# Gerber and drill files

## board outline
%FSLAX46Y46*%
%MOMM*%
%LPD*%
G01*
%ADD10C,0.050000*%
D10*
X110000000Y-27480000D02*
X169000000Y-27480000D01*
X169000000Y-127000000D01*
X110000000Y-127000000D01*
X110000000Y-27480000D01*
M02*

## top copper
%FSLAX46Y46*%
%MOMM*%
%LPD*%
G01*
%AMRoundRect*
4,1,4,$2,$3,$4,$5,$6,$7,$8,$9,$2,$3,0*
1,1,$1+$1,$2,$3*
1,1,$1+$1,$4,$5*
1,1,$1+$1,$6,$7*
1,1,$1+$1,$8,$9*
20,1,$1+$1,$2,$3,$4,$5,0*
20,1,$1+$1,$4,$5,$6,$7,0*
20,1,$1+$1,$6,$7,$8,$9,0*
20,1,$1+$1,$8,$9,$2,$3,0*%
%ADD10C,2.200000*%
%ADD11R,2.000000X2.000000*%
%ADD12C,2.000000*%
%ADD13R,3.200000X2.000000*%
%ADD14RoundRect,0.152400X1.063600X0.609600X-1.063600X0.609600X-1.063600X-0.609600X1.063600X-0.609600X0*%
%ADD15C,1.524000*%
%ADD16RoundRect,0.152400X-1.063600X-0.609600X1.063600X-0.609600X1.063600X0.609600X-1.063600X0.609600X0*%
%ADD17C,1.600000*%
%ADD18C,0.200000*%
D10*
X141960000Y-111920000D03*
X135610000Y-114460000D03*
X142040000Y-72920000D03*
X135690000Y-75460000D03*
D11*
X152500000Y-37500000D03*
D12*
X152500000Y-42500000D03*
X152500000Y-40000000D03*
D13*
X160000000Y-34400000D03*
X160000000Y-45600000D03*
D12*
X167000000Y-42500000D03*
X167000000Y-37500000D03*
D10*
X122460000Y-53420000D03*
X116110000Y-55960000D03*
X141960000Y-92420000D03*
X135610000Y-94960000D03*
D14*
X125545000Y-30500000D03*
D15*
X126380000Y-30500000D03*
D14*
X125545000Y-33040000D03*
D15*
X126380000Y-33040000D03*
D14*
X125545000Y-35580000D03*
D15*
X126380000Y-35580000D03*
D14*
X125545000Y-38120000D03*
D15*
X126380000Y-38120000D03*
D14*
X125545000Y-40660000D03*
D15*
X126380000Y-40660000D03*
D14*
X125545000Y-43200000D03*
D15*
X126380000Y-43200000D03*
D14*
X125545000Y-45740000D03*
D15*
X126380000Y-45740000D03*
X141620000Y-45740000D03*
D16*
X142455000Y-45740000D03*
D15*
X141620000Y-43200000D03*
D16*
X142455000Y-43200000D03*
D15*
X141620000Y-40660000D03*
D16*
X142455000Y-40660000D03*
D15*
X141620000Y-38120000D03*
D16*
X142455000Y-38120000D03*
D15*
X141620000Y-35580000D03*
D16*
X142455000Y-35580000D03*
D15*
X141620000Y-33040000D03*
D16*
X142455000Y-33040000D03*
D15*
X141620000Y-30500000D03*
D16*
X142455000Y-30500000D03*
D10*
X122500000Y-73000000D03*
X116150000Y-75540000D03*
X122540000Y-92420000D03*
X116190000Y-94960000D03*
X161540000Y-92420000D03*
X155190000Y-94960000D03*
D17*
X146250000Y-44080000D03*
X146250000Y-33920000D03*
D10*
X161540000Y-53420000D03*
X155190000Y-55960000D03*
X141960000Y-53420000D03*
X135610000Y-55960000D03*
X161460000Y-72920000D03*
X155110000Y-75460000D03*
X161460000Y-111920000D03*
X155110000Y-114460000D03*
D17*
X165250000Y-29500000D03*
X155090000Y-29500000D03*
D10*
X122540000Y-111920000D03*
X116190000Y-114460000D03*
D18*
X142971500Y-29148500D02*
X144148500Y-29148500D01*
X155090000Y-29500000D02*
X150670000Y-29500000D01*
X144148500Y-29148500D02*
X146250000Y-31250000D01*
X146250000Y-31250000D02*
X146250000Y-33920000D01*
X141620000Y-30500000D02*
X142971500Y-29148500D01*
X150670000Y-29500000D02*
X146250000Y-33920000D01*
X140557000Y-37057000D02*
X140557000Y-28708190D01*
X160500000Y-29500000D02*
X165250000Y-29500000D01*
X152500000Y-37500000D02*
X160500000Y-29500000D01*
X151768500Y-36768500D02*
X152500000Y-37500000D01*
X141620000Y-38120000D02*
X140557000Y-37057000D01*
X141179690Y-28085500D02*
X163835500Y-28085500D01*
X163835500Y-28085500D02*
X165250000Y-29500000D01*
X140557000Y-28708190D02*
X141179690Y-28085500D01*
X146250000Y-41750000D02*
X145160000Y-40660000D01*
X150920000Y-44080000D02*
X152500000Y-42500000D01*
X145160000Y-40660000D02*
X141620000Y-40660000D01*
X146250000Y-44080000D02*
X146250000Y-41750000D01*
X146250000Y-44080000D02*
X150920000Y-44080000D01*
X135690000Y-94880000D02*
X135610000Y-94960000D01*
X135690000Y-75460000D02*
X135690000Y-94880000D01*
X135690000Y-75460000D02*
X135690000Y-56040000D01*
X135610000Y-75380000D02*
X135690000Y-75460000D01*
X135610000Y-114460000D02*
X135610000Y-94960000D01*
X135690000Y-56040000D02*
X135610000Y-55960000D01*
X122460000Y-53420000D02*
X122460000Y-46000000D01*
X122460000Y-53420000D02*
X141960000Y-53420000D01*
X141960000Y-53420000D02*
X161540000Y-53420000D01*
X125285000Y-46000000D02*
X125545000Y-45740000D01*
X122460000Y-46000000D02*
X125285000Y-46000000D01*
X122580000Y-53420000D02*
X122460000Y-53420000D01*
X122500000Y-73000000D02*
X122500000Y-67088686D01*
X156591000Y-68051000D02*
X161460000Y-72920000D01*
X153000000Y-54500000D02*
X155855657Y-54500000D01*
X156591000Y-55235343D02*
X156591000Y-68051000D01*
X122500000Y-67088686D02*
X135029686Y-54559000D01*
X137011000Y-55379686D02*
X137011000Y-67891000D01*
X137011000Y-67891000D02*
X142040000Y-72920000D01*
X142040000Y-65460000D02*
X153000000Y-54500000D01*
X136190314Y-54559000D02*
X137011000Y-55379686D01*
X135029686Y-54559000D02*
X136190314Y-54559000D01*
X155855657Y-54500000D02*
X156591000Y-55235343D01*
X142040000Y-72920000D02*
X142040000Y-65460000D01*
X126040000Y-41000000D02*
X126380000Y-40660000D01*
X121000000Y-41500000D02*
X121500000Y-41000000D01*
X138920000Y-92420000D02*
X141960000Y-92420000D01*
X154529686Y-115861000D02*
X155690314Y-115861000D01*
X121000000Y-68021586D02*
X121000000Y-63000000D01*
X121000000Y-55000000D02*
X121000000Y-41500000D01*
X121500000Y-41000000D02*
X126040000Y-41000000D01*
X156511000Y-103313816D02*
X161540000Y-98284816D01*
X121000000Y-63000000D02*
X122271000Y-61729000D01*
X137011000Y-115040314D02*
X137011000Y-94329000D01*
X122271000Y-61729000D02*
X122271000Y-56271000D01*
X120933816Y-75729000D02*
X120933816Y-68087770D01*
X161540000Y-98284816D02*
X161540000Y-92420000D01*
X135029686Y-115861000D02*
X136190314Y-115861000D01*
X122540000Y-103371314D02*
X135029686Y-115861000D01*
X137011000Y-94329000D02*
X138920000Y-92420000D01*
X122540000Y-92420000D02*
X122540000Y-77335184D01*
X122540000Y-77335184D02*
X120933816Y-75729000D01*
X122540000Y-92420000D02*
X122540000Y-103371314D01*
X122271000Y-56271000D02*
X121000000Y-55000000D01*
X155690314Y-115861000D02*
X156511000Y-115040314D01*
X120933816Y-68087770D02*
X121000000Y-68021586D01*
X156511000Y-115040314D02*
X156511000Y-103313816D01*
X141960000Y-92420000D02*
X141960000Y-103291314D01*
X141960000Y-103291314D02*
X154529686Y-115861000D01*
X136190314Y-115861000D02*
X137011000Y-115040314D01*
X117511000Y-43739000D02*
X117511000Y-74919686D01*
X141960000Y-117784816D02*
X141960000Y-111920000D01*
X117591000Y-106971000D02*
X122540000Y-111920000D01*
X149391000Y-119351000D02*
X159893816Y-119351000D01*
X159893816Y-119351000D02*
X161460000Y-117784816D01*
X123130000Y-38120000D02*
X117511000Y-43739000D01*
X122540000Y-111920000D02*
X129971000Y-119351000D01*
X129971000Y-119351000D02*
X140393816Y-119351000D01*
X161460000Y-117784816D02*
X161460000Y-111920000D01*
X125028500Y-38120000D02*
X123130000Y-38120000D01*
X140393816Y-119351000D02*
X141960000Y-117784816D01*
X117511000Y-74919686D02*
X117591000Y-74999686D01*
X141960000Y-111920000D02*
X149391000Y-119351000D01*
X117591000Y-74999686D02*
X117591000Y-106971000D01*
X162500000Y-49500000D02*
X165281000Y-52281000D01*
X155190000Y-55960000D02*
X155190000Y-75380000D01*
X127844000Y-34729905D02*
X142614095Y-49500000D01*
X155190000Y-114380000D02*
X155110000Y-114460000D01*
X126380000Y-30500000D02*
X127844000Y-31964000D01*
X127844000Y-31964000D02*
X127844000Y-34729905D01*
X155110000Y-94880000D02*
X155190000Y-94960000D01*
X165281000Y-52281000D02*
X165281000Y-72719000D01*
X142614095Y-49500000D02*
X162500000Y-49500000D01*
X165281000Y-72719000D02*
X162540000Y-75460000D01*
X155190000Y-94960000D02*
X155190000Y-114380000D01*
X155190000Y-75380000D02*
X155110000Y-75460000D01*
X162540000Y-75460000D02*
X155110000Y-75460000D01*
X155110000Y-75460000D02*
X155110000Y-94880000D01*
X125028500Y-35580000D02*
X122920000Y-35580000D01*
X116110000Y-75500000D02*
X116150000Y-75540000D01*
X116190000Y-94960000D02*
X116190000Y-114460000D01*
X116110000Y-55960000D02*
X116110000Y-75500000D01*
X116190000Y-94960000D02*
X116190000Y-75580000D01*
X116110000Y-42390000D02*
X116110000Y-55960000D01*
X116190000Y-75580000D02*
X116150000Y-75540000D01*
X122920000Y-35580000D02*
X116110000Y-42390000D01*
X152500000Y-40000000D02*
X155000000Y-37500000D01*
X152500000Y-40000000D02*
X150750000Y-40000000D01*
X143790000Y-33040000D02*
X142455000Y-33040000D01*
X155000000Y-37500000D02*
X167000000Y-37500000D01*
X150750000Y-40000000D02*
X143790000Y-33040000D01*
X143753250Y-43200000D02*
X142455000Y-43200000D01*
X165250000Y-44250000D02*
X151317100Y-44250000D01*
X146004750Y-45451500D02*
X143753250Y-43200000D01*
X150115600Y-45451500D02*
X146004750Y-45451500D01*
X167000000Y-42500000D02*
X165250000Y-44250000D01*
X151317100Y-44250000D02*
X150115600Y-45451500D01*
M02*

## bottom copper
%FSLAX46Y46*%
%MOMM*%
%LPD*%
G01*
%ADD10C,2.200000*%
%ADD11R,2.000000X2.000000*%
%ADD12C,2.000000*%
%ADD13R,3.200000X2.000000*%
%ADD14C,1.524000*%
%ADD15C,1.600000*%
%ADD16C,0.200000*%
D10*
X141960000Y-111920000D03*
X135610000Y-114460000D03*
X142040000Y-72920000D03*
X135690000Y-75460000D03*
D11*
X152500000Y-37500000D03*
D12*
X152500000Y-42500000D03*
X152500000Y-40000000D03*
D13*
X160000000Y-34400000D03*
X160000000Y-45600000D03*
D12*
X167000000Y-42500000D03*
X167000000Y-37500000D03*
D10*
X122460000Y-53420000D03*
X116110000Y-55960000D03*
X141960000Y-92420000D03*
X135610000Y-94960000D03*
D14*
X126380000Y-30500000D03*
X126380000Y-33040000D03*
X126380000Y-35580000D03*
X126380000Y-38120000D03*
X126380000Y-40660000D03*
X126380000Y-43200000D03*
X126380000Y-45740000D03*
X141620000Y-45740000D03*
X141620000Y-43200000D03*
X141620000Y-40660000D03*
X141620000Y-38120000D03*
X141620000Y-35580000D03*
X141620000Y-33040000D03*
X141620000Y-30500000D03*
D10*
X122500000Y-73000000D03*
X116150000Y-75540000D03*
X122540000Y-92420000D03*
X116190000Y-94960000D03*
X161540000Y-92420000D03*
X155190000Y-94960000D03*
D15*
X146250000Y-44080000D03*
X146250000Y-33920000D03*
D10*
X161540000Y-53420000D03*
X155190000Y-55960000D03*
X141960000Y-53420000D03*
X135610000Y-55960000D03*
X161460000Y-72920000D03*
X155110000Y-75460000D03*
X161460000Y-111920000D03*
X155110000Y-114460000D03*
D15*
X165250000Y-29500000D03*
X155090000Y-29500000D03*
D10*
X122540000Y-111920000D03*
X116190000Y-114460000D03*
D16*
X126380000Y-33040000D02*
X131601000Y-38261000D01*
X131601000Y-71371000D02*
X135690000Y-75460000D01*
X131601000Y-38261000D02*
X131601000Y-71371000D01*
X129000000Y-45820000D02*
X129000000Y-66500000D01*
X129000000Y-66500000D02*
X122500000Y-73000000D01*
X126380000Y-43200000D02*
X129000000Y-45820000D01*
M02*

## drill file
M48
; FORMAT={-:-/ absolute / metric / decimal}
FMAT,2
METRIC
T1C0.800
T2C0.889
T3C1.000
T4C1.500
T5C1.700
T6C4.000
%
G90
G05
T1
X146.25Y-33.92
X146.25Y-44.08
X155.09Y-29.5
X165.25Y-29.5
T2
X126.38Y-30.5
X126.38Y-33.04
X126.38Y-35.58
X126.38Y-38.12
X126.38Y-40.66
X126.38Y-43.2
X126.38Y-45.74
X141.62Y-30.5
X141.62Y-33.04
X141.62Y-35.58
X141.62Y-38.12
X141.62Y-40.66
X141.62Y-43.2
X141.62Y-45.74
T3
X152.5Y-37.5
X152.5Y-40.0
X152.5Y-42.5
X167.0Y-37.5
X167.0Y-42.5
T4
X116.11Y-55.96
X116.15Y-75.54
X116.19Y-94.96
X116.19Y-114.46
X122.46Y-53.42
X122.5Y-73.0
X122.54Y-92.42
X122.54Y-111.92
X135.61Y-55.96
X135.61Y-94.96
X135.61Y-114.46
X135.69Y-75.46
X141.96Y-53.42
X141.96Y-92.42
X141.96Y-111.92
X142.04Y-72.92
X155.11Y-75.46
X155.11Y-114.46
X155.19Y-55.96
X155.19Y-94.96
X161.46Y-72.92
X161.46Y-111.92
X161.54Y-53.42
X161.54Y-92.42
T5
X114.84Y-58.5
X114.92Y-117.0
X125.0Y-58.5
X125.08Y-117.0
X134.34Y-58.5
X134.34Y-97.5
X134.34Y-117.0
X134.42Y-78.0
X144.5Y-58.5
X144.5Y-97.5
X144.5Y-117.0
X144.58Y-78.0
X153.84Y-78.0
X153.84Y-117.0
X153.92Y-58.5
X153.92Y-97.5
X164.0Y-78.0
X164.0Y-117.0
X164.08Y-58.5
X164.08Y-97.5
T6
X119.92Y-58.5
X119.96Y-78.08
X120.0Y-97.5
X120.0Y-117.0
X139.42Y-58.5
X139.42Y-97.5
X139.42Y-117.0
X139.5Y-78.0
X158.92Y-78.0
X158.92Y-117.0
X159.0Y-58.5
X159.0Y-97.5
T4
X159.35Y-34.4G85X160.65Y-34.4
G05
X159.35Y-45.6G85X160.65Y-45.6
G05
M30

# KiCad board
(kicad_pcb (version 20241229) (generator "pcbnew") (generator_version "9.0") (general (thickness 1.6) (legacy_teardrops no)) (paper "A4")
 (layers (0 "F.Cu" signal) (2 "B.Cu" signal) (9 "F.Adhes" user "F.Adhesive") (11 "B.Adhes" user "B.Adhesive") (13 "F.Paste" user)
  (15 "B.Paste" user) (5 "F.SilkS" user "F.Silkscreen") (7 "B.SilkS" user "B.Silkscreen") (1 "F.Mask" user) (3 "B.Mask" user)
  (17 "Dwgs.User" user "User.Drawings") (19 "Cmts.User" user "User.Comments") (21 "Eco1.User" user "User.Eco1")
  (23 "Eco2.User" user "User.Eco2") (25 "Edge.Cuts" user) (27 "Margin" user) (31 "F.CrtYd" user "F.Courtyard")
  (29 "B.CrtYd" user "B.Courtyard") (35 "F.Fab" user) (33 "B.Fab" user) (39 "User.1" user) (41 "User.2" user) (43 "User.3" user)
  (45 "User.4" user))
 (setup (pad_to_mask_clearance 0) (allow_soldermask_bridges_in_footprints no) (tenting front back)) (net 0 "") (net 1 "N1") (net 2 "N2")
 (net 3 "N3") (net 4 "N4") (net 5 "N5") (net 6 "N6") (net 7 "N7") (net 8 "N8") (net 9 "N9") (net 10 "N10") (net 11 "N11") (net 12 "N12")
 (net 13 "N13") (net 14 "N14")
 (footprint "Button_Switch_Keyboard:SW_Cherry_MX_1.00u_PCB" (layer "F.Cu") (at 141.96 111.92)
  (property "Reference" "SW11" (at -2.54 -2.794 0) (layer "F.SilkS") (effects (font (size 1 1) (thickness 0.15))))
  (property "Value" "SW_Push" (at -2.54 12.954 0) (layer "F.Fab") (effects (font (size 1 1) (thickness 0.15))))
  (pad "" np_thru_hole circle (at -7.62 5.08) (size 1.7 1.7) (drill 1.7) (layers "*.Cu" "*.Mask"))
  (pad "" np_thru_hole circle (at -2.54 5.08) (size 4 4) (drill 4) (layers "*.Cu" "*.Mask"))
  (pad "" np_thru_hole circle (at 2.54 5.08) (size 1.7 1.7) (drill 1.7) (layers "*.Cu" "*.Mask"))
  (pad "1" thru_hole circle (at 0 0) (size 2.2 2.2) (drill 1.5) (layers "*.Cu" "*.Mask") (remove_unused_layers no) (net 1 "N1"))
  (pad "2" thru_hole circle (at -6.35 2.54) (size 2.2 2.2) (drill 1.5) (layers "*.Cu" "*.Mask") (remove_unused_layers no) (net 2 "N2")))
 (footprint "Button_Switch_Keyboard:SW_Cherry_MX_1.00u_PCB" (layer "F.Cu") (at 142.04 72.92)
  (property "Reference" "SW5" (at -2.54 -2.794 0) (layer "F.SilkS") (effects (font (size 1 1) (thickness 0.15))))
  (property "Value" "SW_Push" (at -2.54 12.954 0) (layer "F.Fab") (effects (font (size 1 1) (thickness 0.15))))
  (pad "" np_thru_hole circle (at -7.62 5.08) (size 1.7 1.7) (drill 1.7) (layers "*.Cu" "*.Mask"))
  (pad "" np_thru_hole circle (at -2.54 5.08) (size 4 4) (drill 4) (layers "*.Cu" "*.Mask"))
  (pad "" np_thru_hole circle (at 2.54 5.08) (size 1.7 1.7) (drill 1.7) (layers "*.Cu" "*.Mask"))
  (pad "1" thru_hole circle (at 0 0) (size 2.2 2.2) (drill 1.5) (layers "*.Cu" "*.Mask") (remove_unused_layers no) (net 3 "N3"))
  (pad "2" thru_hole circle (at -6.35 2.54) (size 2.2 2.2) (drill 1.5) (layers "*.Cu" "*.Mask") (remove_unused_layers no) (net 2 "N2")))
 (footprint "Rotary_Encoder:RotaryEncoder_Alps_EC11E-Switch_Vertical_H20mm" (layer "F.Cu") (at 152.5 37.5)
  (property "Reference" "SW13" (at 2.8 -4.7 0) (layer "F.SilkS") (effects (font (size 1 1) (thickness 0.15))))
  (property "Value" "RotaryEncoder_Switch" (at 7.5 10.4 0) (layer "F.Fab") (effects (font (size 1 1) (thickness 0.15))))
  (pad "A" thru_hole rect (at 0 0) (size 2 2) (drill 1) (layers "*.Cu" "*.Mask") (remove_unused_layers no) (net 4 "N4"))
  (pad "B" thru_hole circle (at 0 5) (size 2 2) (drill 1) (layers "*.Cu" "*.Mask") (remove_unused_layers no) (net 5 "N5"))
  (pad "C" thru_hole circle (at 0 2.5) (size 2 2) (drill 1) (layers "*.Cu" "*.Mask") (remove_unused_layers no) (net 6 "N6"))
  (pad "MP" thru_hole rect (at 7.5 -3.1) (size 3.2 2) (drill oval 2.8 1.5) (layers "*.Cu" "*.Mask") (remove_unused_layers no))
  (pad "MP" thru_hole rect (at 7.5 8.1) (size 3.2 2) (drill oval 2.8 1.5) (layers "*.Cu" "*.Mask") (remove_unused_layers no))
  (pad "S1" thru_hole circle (at 14.5 5) (size 2 2) (drill 1) (layers "*.Cu" "*.Mask") (remove_unused_layers no) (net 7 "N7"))
  (pad "S2" thru_hole circle (at 14.5 0) (size 2 2) (drill 1) (layers "*.Cu" "*.Mask") (remove_unused_layers no) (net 6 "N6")))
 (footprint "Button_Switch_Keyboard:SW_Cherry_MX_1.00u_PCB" (layer "F.Cu") (at 122.46 53.42)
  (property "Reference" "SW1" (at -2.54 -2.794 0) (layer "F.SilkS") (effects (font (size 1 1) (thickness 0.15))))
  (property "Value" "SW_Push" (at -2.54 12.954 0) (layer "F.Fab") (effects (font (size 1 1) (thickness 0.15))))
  (pad "" np_thru_hole circle (at -7.62 5.08) (size 1.7 1.7) (drill 1.7) (layers "*.Cu" "*.Mask"))
  (pad "" np_thru_hole circle (at -2.54 5.08) (size 4 4) (drill 4) (layers "*.Cu" "*.Mask"))
  (pad "" np_thru_hole circle (at 2.54 5.08) (size 1.7 1.7) (drill 1.7) (layers "*.Cu" "*.Mask"))
  (pad "1" thru_hole circle (at 0 0) (size 2.2 2.2) (drill 1.5) (layers "*.Cu" "*.Mask") (remove_unused_layers no) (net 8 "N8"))
  (pad "2" thru_hole circle (at -6.35 2.54) (size 2.2 2.2) (drill 1.5) (layers "*.Cu" "*.Mask") (remove_unused_layers no) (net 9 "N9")))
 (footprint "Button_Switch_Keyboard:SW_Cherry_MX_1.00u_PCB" (layer "F.Cu") (at 141.96 92.42)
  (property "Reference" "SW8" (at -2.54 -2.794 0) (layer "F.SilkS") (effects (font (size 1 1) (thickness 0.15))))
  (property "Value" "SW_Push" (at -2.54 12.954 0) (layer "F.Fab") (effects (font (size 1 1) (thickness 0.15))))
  (pad "" np_thru_hole circle (at -7.62 5.08) (size 1.7 1.7) (drill 1.7) (layers "*.Cu" "*.Mask"))
  (pad "" np_thru_hole circle (at -2.54 5.08) (size 4 4) (drill 4) (layers "*.Cu" "*.Mask"))
  (pad "" np_thru_hole circle (at 2.54 5.08) (size 1.7 1.7) (drill 1.7) (layers "*.Cu" "*.Mask"))
  (pad "1" thru_hole circle (at 0 0) (size 2.2 2.2) (drill 1.5) (layers "*.Cu" "*.Mask") (remove_unused_layers no) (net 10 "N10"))
  (pad "2" thru_hole circle (at -6.35 2.54) (size 2.2 2.2) (drill 1.5) (layers "*.Cu" "*.Mask") (remove_unused_layers no) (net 2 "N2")))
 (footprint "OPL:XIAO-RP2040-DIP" (layer "F.Cu") (at 134 38.12)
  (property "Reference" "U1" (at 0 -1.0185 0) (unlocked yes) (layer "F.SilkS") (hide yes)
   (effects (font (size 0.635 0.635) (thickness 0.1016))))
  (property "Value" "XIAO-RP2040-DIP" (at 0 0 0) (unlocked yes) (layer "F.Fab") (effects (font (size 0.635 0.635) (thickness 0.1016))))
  (pad "1" smd roundrect (at -8.455 -7.62 180) (size 2.432 1.524) (layers "F.Cu" "F.Mask") (roundrect_rratio 0.1) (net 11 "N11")
   (thermal_bridge_angle 45))
  (pad "1" thru_hole circle (at -7.62 -7.62 180) (size 1.524 1.524) (drill 0.889) (layers "*.Cu" "*.Mask") (remove_unused_layers no)
   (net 11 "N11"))
  (pad "2" smd roundrect (at -8.455 -5.08 180) (size 2.432 1.524) (layers "F.Cu" "F.Mask") (roundrect_rratio 0.1) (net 2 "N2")
   (thermal_bridge_angle 45))
  (pad "2" thru_hole circle (at -7.62 -5.08 180) (size 1.524 1.524) (drill 0.889) (layers "*.Cu" "*.Mask") (remove_unused_layers no)
   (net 2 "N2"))
  (pad "3" smd roundrect (at -8.455 -2.54 180) (size 2.432 1.524) (layers "F.Cu" "F.Mask") (roundrect_rratio 0.1) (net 9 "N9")
   (thermal_bridge_angle 45))
  (pad "3" thru_hole circle (at -7.62 -2.54 180) (size 1.524 1.524) (drill 0.889) (layers "*.Cu" "*.Mask") (remove_unused_layers no)
   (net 9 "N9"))
  (pad "4" smd roundrect (at -8.455 0 180) (size 2.432 1.524) (layers "F.Cu" "F.Mask") (roundrect_rratio 0.1) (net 1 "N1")
   (thermal_bridge_angle 45))
  (pad "4" thru_hole circle (at -7.62 0 180) (size 1.524 1.524) (drill 0.889) (layers "*.Cu" "*.Mask") (remove_unused_layers no)
   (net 1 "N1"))
  (pad "5" smd roundrect (at -8.455 2.54 180) (size 2.432 1.524) (layers "F.Cu" "F.Mask") (roundrect_rratio 0.1) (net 10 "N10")
   (thermal_bridge_angle 45))
  (pad "5" thru_hole circle (at -7.62 2.54 180) (size 1.524 1.524) (drill 0.889) (layers "*.Cu" "*.Mask") (remove_unused_layers no)
   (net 10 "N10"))
  (pad "6" smd roundrect (at -8.455 5.08 180) (size 2.432 1.524) (layers "F.Cu" "F.Mask") (roundrect_rratio 0.1) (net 3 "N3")
   (thermal_bridge_angle 45))
  (pad "6" thru_hole circle (at -7.62 5.08 180) (size 1.524 1.524) (drill 0.889) (layers "*.Cu" "*.Mask") (remove_unused_layers no)
   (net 3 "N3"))
  (pad "7" smd roundrect (at -8.455 7.62 180) (size 2.432 1.524) (layers "F.Cu" "F.Mask") (roundrect_rratio 0.1) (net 8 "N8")
   (thermal_bridge_angle 45))
  (pad "7" thru_hole circle (at -7.62 7.62 180) (size 1.524 1.524) (drill 0.889) (layers "*.Cu" "*.Mask") (remove_unused_layers no)
   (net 8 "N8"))
  (pad "8" thru_hole circle (at 7.62 7.62) (size 1.524 1.524) (drill 0.889) (layers "*.Cu" "*.Mask") (remove_unused_layers no)
   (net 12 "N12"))
  (pad "8" smd roundrect (at 8.455 7.62) (size 2.432 1.524) (layers "F.Cu" "F.Mask") (roundrect_rratio 0.1) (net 12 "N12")
   (thermal_bridge_angle 45))
  (pad "9" thru_hole circle (at 7.62 5.08) (size 1.524 1.524) (drill 0.889) (layers "*.Cu" "*.Mask") (remove_unused_layers no) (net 7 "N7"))
  (pad "9" smd roundrect (at 8.455 5.08) (size 2.432 1.524) (layers "F.Cu" "F.Mask") (roundrect_rratio 0.1) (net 7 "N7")
   (thermal_bridge_angle 45))
  (pad "10" thru_hole circle (at 7.62 2.54) (size 1.524 1.524) (drill 0.889) (layers "*.Cu" "*.Mask") (remove_unused_layers no) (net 5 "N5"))
  (pad "10" smd roundrect (at 8.455 2.54) (size 2.432 1.524) (layers "F.Cu" "F.Mask") (roundrect_rratio 0.1) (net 5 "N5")
   (thermal_bridge_angle 45))
  (pad "11" thru_hole circle (at 7.62 0) (size 1.524 1.524) (drill 0.889) (layers "*.Cu" "*.Mask") (remove_unused_layers no) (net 4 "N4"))
  (pad "11" smd roundrect (at 8.455 0) (size 2.432 1.524) (layers "F.Cu" "F.Mask") (roundrect_rratio 0.1) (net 4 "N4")
   (thermal_bridge_angle 45))
  (pad "12" thru_hole circle (at 7.62 -2.54) (size 1.524 1.524) (drill 0.889) (layers "*.Cu" "*.Mask") (remove_unused_layers no)
   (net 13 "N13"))
  (pad "12" smd roundrect (at 8.455 -2.54) (size 2.432 1.524) (layers "F.Cu" "F.Mask") (roundrect_rratio 0.1) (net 13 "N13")
   (thermal_bridge_angle 45))
  (pad "13" thru_hole circle (at 7.62 -5.08) (size 1.524 1.524) (drill 0.889) (layers "*.Cu" "*.Mask") (remove_unused_layers no)
   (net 6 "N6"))
  (pad "13" smd roundrect (at 8.455 -5.08) (size 2.432 1.524) (layers "F.Cu" "F.Mask") (roundrect_rratio 0.1) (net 6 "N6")
   (thermal_bridge_angle 45))
  (pad "14" thru_hole circle (at 7.62 -7.62) (size 1.524 1.524) (drill 0.889) (layers "*.Cu" "*.Mask") (remove_unused_layers no)
   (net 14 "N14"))
  (pad "14" smd roundrect (at 8.455 -7.62) (size 2.432 1.524) (layers "F.Cu" "F.Mask") (roundrect_rratio 0.1) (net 14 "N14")
   (thermal_bridge_angle 45)))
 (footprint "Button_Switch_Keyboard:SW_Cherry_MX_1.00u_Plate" (layer "F.Cu") (at 122.5 73)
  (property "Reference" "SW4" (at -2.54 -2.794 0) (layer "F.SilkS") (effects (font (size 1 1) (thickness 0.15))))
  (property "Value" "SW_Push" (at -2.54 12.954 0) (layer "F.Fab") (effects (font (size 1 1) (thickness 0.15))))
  (pad "" np_thru_hole circle (at -2.54 5.08) (size 4 4) (drill 4) (layers "*.Cu" "*.Mask"))
  (pad "1" thru_hole circle (at 0 0) (size 2.2 2.2) (drill 1.5) (layers "*.Cu" "*.Mask") (remove_unused_layers no) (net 3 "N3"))
  (pad "2" thru_hole circle (at -6.35 2.54) (size 2.2 2.2) (drill 1.5) (layers "*.Cu" "*.Mask") (remove_unused_layers no) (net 9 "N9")))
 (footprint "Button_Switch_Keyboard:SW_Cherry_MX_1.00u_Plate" (layer "F.Cu") (at 122.54 92.42)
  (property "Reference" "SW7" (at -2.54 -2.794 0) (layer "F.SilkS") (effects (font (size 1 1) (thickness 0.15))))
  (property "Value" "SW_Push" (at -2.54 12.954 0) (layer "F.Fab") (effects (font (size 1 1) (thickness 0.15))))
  (pad "" np_thru_hole circle (at -2.54 5.08) (size 4 4) (drill 4) (layers "*.Cu" "*.Mask"))
  (pad "1" thru_hole circle (at 0 0) (size 2.2 2.2) (drill 1.5) (layers "*.Cu" "*.Mask") (remove_unused_layers no) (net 10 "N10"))
  (pad "2" thru_hole circle (at -6.35 2.54) (size 2.2 2.2) (drill 1.5) (layers "*.Cu" "*.Mask") (remove_unused_layers no) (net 9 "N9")))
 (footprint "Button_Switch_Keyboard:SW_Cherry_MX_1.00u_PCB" (layer "F.Cu") (at 161.54 92.42)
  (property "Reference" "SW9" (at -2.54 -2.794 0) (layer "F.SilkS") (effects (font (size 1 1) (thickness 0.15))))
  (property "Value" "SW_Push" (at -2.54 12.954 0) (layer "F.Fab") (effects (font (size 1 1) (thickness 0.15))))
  (pad "" np_thru_hole circle (at -7.62 5.08) (size 1.7 1.7) (drill 1.7) (layers "*.Cu" "*.Mask"))
  (pad "" np_thru_hole circle (at -2.54 5.08) (size 4 4) (drill 4) (layers "*.Cu" "*.Mask"))
  (pad "" np_thru_hole circle (at 2.54 5.08) (size 1.7 1.7) (drill 1.7) (layers "*.Cu" "*.Mask"))
  (pad "1" thru_hole circle (at 0 0) (size 2.2 2.2) (drill 1.5) (layers "*.Cu" "*.Mask") (remove_unused_layers no) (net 10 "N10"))
  (pad "2" thru_hole circle (at -6.35 2.54) (size 2.2 2.2) (drill 1.5) (layers "*.Cu" "*.Mask") (remove_unused_layers no) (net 11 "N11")))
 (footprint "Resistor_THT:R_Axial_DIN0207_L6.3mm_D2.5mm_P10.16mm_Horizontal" (layer "F.Cu") (at 146.25 44.08 90)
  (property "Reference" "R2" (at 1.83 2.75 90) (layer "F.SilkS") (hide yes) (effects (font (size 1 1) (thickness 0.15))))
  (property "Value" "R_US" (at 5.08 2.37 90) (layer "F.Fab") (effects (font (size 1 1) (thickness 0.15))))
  (pad "1" thru_hole circle (at 0 0 90) (size 1.6 1.6) (drill 0.8) (layers "*.Cu" "*.Mask") (remove_unused_layers no) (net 5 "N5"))
  (pad "2" thru_hole circle (at 10.16 0 90) (size 1.6 1.6) (drill 0.8) (layers "*.Cu" "*.Mask") (remove_unused_layers no) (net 14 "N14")))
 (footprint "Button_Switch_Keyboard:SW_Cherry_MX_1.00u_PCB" (layer "F.Cu") (at 161.54 53.42)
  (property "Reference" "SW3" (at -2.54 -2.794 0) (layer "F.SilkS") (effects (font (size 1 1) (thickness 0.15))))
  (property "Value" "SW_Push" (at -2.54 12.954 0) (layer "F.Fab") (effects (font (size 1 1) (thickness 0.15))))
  (pad "" np_thru_hole circle (at -7.62 5.08) (size 1.7 1.7) (drill 1.7) (layers "*.Cu" "*.Mask"))
  (pad "" np_thru_hole circle (at -2.54 5.08) (size 4 4) (drill 4) (layers "*.Cu" "*.Mask"))
  (pad "" np_thru_hole circle (at 2.54 5.08) (size 1.7 1.7) (drill 1.7) (layers "*.Cu" "*.Mask"))
  (pad "1" thru_hole circle (at 0 0) (size 2.2 2.2) (drill 1.5) (layers "*.Cu" "*.Mask") (remove_unused_layers no) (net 8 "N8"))
  (pad "2" thru_hole circle (at -6.35 2.54) (size 2.2 2.2) (drill 1.5) (layers "*.Cu" "*.Mask") (remove_unused_layers no) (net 11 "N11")))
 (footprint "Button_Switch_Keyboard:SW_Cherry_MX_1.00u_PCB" (layer "F.Cu") (at 141.96 53.42)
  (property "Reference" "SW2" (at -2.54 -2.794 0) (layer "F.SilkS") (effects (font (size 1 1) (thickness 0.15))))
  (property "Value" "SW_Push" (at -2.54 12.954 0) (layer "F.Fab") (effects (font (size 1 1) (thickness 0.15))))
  (pad "" np_thru_hole circle (at -7.62 5.08) (size 1.7 1.7) (drill 1.7) (layers "*.Cu" "*.Mask"))
  (pad "" np_thru_hole circle (at -2.54 5.08) (size 4 4) (drill 4) (layers "*.Cu" "*.Mask"))
  (pad "" np_thru_hole circle (at 2.54 5.08) (size 1.7 1.7) (drill 1.7) (layers "*.Cu" "*.Mask"))
  (pad "1" thru_hole circle (at 0 0) (size 2.2 2.2) (drill 1.5) (layers "*.Cu" "*.Mask") (remove_unused_layers no) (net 8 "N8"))
  (pad "2" thru_hole circle (at -6.35 2.54) (size 2.2 2.2) (drill 1.5) (layers "*.Cu" "*.Mask") (remove_unused_layers no) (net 2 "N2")))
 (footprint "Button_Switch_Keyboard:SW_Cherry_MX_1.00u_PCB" (layer "F.Cu") (at 161.46 72.92)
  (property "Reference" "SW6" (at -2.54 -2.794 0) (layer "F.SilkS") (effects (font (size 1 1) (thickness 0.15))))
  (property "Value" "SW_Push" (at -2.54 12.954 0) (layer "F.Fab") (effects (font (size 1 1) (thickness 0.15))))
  (pad "" np_thru_hole circle (at -7.62 5.08) (size 1.7 1.7) (drill 1.7) (layers "*.Cu" "*.Mask"))
  (pad "" np_thru_hole circle (at -2.54 5.08) (size 4 4) (drill 4) (layers "*.Cu" "*.Mask"))
  (pad "" np_thru_hole circle (at 2.54 5.08) (size 1.7 1.7) (drill 1.7) (layers "*.Cu" "*.Mask"))
  (pad "1" thru_hole circle (at 0 0) (size 2.2 2.2) (drill 1.5) (layers "*.Cu" "*.Mask") (remove_unused_layers no) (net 3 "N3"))
  (pad "2" thru_hole circle (at -6.35 2.54) (size 2.2 2.2) (drill 1.5) (layers "*.Cu" "*.Mask") (remove_unused_layers no) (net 11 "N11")))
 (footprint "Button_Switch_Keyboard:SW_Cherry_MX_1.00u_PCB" (layer "F.Cu") (at 161.46 111.92)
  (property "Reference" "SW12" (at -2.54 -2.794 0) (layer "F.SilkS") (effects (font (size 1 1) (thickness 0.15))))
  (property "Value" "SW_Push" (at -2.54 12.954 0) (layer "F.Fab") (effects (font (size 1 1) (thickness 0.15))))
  (pad "" np_thru_hole circle (at -7.62 5.08) (size 1.7 1.7) (drill 1.7) (layers "*.Cu" "*.Mask"))
  (pad "" np_thru_hole circle (at -2.54 5.08) (size 4 4) (drill 4) (layers "*.Cu" "*.Mask"))
  (pad "" np_thru_hole circle (at 2.54 5.08) (size 1.7 1.7) (drill 1.7) (layers "*.Cu" "*.Mask"))
  (pad "1" thru_hole circle (at 0 0) (size 2.2 2.2) (drill 1.5) (layers "*.Cu" "*.Mask") (remove_unused_layers no) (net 1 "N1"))
  (pad "2" thru_hole circle (at -6.35 2.54) (size 2.2 2.2) (drill 1.5) (layers "*.Cu" "*.Mask") (remove_unused_layers no) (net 11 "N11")))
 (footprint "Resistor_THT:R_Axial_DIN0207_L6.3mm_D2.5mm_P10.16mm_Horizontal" (layer "F.Cu") (at 165.25 29.5 180)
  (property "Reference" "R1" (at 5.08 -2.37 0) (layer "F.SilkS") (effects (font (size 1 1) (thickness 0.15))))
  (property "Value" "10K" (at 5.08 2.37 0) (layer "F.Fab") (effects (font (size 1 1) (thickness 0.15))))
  (pad "1" thru_hole circle (at 0 0 180) (size 1.6 1.6) (drill 0.8) (layers "*.Cu" "*.Mask") (remove_unused_layers no) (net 4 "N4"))
  (pad "2" thru_hole circle (at 10.16 0 180) (size 1.6 1.6) (drill 0.8) (layers "*.Cu" "*.Mask") (remove_unused_layers no) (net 14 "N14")))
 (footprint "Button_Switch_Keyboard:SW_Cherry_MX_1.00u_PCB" (layer "F.Cu") (at 122.54 111.92)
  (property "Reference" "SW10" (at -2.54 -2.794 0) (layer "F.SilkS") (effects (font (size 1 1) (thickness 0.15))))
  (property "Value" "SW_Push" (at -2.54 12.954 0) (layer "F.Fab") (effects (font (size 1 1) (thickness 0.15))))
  (pad "" np_thru_hole circle (at -7.62 5.08) (size 1.7 1.7) (drill 1.7) (layers "*.Cu" "*.Mask"))
  (pad "" np_thru_hole circle (at -2.54 5.08) (size 4 4) (drill 4) (layers "*.Cu" "*.Mask"))
  (pad "" np_thru_hole circle (at 2.54 5.08) (size 1.7 1.7) (drill 1.7) (layers "*.Cu" "*.Mask"))
  (pad "1" thru_hole circle (at 0 0) (size 2.2 2.2) (drill 1.5) (layers "*.Cu" "*.Mask") (remove_unused_layers no) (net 1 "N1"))
  (pad "2" thru_hole circle (at -6.35 2.54) (size 2.2 2.2) (drill 1.5) (layers "*.Cu" "*.Mask") (remove_unused_layers no) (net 9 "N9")))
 (gr_rect (start 110 27.48) (end 169 127) (stroke (width 0.05) (type default)) (fill no) (layer "Edge.Cuts"))
 (segment (start 142.9715 29.1485) (end 144.1485 29.1485) (width 0.2) (layer "F.Cu") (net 14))
 (segment (start 155.09 29.5) (end 150.67 29.5) (width 0.2) (layer "F.Cu") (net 14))
 (segment (start 144.1485 29.1485) (end 146.25 31.25) (width 0.2) (layer "F.Cu") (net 14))
 (segment (start 146.25 31.25) (end 146.25 33.92) (width 0.2) (layer "F.Cu") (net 14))
 (segment (start 141.62 30.5) (end 142.9715 29.1485) (width 0.2) (layer "F.Cu") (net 14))
 (segment (start 150.67 29.5) (end 146.25 33.92) (width 0.2) (layer "F.Cu") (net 14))
 (segment (start 140.557 37.057) (end 140.557 28.70819) (width 0.2) (layer "F.Cu") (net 4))
 (segment (start 160.5 29.5) (end 165.25 29.5) (width 0.2) (layer "F.Cu") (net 4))
 (segment (start 152.5 37.5) (end 160.5 29.5) (width 0.2) (layer "F.Cu") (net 4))
 (segment (start 151.7685 36.7685) (end 152.5 37.5) (width 0.2) (layer "F.Cu") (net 4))
 (segment (start 141.62 38.12) (end 140.557 37.057) (width 0.2) (layer "F.Cu") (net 4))
 (segment (start 141.17969 28.0855) (end 163.8355 28.0855) (width 0.2) (layer "F.Cu") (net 4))
 (segment (start 163.8355 28.0855) (end 165.25 29.5) (width 0.2) (layer "F.Cu") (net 4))
 (segment (start 140.557 28.70819) (end 141.17969 28.0855) (width 0.2) (layer "F.Cu") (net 4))
 (segment (start 146.25 41.75) (end 145.16 40.66) (width 0.2) (layer "F.Cu") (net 5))
 (segment (start 150.92 44.08) (end 152.5 42.5) (width 0.2) (layer "F.Cu") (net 5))
 (segment (start 145.16 40.66) (end 141.62 40.66) (width 0.2) (layer "F.Cu") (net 5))
 (segment (start 146.25 44.08) (end 146.25 41.75) (width 0.2) (layer "F.Cu") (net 5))
 (segment (start 146.25 44.08) (end 150.92 44.08) (width 0.2) (layer "F.Cu") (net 5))
 (segment (start 135.69 94.88) (end 135.61 94.96) (width 0.2) (layer "F.Cu") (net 2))
 (segment (start 135.69 75.46) (end 135.69 94.88) (width 0.2) (layer "F.Cu") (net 2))
 (segment (start 135.69 75.46) (end 135.69 56.04) (width 0.2) (layer "F.Cu") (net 2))
 (segment (start 135.61 75.38) (end 135.69 75.46) (width 0.2) (layer "F.Cu") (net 2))
 (segment (start 135.61 114.46) (end 135.61 94.96) (width 0.2) (layer "F.Cu") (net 2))
 (segment (start 135.69 56.04) (end 135.61 55.96) (width 0.2) (layer "F.Cu") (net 2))
 (segment (start 126.38 33.04) (end 131.601 38.261) (width 0.2) (layer "B.Cu") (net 2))
 (segment (start 131.601 71.371) (end 135.69 75.46) (width 0.2) (layer "B.Cu") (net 2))
 (segment (start 131.601 38.261) (end 131.601 71.371) (width 0.2) (layer "B.Cu") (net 2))
 (segment (start 122.46 53.42) (end 122.46 46) (width 0.2) (layer "F.Cu") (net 8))
 (segment (start 122.46 53.42) (end 141.96 53.42) (width 0.2) (layer "F.Cu") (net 8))
 (segment (start 141.96 53.42) (end 161.54 53.42) (width 0.2) (layer "F.Cu") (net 8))
 (segment (start 125.285 46) (end 125.545 45.74) (width 0.2) (layer "F.Cu") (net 8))
 (segment (start 122.46 46) (end 125.285 46) (width 0.2) (layer "F.Cu") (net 8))
 (segment (start 122.58 53.42) (end 122.46 53.42) (width 0.2) (layer "F.Cu") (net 8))
 (segment (start 122.5 73) (end 122.5 67.088686) (width 0.2) (layer "F.Cu") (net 3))
 (segment (start 156.591 68.051) (end 161.46 72.92) (width 0.2) (layer "F.Cu") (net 3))
 (segment (start 153 54.5) (end 155.855657 54.5) (width 0.2) (layer "F.Cu") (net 3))
 (segment (start 156.591 55.235343) (end 156.591 68.051) (width 0.2) (layer "F.Cu") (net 3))
 (segment (start 122.5 67.088686) (end 135.029686 54.559) (width 0.2) (layer "F.Cu") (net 3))
 (segment (start 137.011 55.379686) (end 137.011 67.891) (width 0.2) (layer "F.Cu") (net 3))
 (segment (start 137.011 67.891) (end 142.04 72.92) (width 0.2) (layer "F.Cu") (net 3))
 (segment (start 142.04 65.46) (end 153 54.5) (width 0.2) (layer "F.Cu") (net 3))
 (segment (start 136.190314 54.559) (end 137.011 55.379686) (width 0.2) (layer "F.Cu") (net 3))
 (segment (start 135.029686 54.559) (end 136.190314 54.559) (width 0.2) (layer "F.Cu") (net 3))
 (segment (start 155.855657 54.5) (end 156.591 55.235343) (width 0.2) (layer "F.Cu") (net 3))
 (segment (start 142.04 72.92) (end 142.04 65.46) (width 0.2) (layer "F.Cu") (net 3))
 (segment (start 129 45.82) (end 129 66.5) (width 0.2) (layer "B.Cu") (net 3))
 (segment (start 129 66.5) (end 122.5 73) (width 0.2) (layer "B.Cu") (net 3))
 (segment (start 126.38 43.2) (end 129 45.82) (width 0.2) (layer "B.Cu") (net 3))
 (segment (start 126.04 41) (end 126.38 40.66) (width 0.2) (layer "F.Cu") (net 10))
 (segment (start 121 41.5) (end 121.5 41) (width 0.2) (layer "F.Cu") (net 10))
 (segment (start 138.92 92.42) (end 141.96 92.42) (width 0.2) (layer "F.Cu") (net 10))
 (segment (start 154.529686 115.861) (end 155.690314 115.861) (width 0.2) (layer "F.Cu") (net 10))
 (segment (start 121 68.021586) (end 121 63) (width 0.2) (layer "F.Cu") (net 10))
 (segment (start 121 55) (end 121 41.5) (width 0.2) (layer "F.Cu") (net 10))
 (segment (start 121.5 41) (end 126.04 41) (width 0.2) (layer "F.Cu") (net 10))
 (segment (start 156.511 103.313816) (end 161.54 98.284816) (width 0.2) (layer "F.Cu") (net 10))
 (segment (start 121 63) (end 122.271 61.729) (width 0.2) (layer "F.Cu") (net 10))
 (segment (start 137.011 115.040314) (end 137.011 94.329) (width 0.2) (layer "F.Cu") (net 10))
 (segment (start 122.271 61.729) (end 122.271 56.271) (width 0.2) (layer "F.Cu") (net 10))
 (segment (start 120.933816 75.729) (end 120.933816 68.08777) (width 0.2) (layer "F.Cu") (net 10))
 (segment (start 161.54 98.284816) (end 161.54 92.42) (width 0.2) (layer "F.Cu") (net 10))
 (segment (start 135.029686 115.861) (end 136.190314 115.861) (width 0.2) (layer "F.Cu") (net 10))
 (segment (start 122.54 103.371314) (end 135.029686 115.861) (width 0.2) (layer "F.Cu") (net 10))
 (segment (start 137.011 94.329) (end 138.92 92.42) (width 0.2) (layer "F.Cu") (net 10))
 (segment (start 122.54 92.42) (end 122.54 77.335184) (width 0.2) (layer "F.Cu") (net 10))
 (segment (start 122.54 77.335184) (end 120.933816 75.729) (width 0.2) (layer "F.Cu") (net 10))
 (segment (start 122.54 92.42) (end 122.54 103.371314) (width 0.2) (layer "F.Cu") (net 10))
 (segment (start 122.271 56.271) (end 121 55) (width 0.2) (layer "F.Cu") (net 10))
 (segment (start 155.690314 115.861) (end 156.511 115.040314) (width 0.2) (layer "F.Cu") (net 10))
 (segment (start 120.933816 68.08777) (end 121 68.021586) (width 0.2) (layer "F.Cu") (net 10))
 (segment (start 156.511 115.040314) (end 156.511 103.313816) (width 0.2) (layer "F.Cu") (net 10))
 (segment (start 141.96 92.42) (end 141.96 103.291314) (width 0.2) (layer "F.Cu") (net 10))
 (segment (start 141.96 103.291314) (end 154.529686 115.861) (width 0.2) (layer "F.Cu") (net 10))
 (segment (start 136.190314 115.861) (end 137.011 115.040314) (width 0.2) (layer "F.Cu") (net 10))
 (segment (start 117.511 43.739) (end 117.511 74.919686) (width 0.2) (layer "F.Cu") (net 1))
 (segment (start 141.96 117.784816) (end 141.96 111.92) (width 0.2) (layer "F.Cu") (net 1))
 (segment (start 117.591 106.971) (end 122.54 111.92) (width 0.2) (layer "F.Cu") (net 1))
 (segment (start 149.391 119.351) (end 159.893816 119.351) (width 0.2) (layer "F.Cu") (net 1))
 (segment (start 159.893816 119.351) (end 161.46 117.784816) (width 0.2) (layer "F.Cu") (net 1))
 (segment (start 123.13 38.12) (end 117.511 43.739) (width 0.2) (layer "F.Cu") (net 1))
 (segment (start 122.54 111.92) (end 129.971 119.351) (width 0.2) (layer "F.Cu") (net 1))
 (segment (start 129.971 119.351) (end 140.393816 119.351) (width 0.2) (layer "F.Cu") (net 1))
 (segment (start 161.46 117.784816) (end 161.46 111.92) (width 0.2) (layer "F.Cu") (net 1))
 (segment (start 125.0285 38.12) (end 123.13 38.12) (width 0.2) (layer "F.Cu") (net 1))
 (segment (start 140.393816 119.351) (end 141.96 117.784816) (width 0.2) (layer "F.Cu") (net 1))
 (segment (start 117.511 74.919686) (end 117.591 74.999686) (width 0.2) (layer "F.Cu") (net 1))
 (segment (start 141.96 111.92) (end 149.391 119.351) (width 0.2) (layer "F.Cu") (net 1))
 (segment (start 117.591 74.999686) (end 117.591 106.971) (width 0.2) (layer "F.Cu") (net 1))
 (segment (start 162.5 49.5) (end 165.281 52.281) (width 0.2) (layer "F.Cu") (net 11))
 (segment (start 155.19 55.96) (end 155.19 75.38) (width 0.2) (layer "F.Cu") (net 11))
 (segment (start 127.844 34.729905) (end 142.614095 49.5) (width 0.2) (layer "F.Cu") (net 11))
 (segment (start 155.19 114.38) (end 155.11 114.46) (width 0.2) (layer "F.Cu") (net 11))
 (segment (start 126.38 30.5) (end 127.844 31.964) (width 0.2) (layer "F.Cu") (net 11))
 (segment (start 127.844 31.964) (end 127.844 34.729905) (width 0.2) (layer "F.Cu") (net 11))
 (segment (start 155.11 94.88) (end 155.19 94.96) (width 0.2) (layer "F.Cu") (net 11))
 (segment (start 165.281 52.281) (end 165.281 72.719) (width 0.2) (layer "F.Cu") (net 11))
 (segment (start 142.614095 49.5) (end 162.5 49.5) (width 0.2) (layer "F.Cu") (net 11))
 (segment (start 165.281 72.719) (end 162.54 75.46) (width 0.2) (layer "F.Cu") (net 11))
 (segment (start 155.19 94.96) (end 155.19 114.38) (width 0.2) (layer "F.Cu") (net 11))
 (segment (start 155.19 75.38) (end 155.11 75.46) (width 0.2) (layer "F.Cu") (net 11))
 (segment (start 162.54 75.46) (end 155.11 75.46) (width 0.2) (layer "F.Cu") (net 11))
 (segment (start 155.11 75.46) (end 155.11 94.88) (width 0.2) (layer "F.Cu") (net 11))
 (segment (start 125.0285 35.58) (end 122.92 35.58) (width 0.2) (layer "F.Cu") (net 9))
 (segment (start 116.11 75.5) (end 116.15 75.54) (width 0.2) (layer "F.Cu") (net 9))
 (segment (start 116.19 94.96) (end 116.19 114.46) (width 0.2) (layer "F.Cu") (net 9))
 (segment (start 116.11 55.96) (end 116.11 75.5) (width 0.2) (layer "F.Cu") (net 9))
 (segment (start 116.19 94.96) (end 116.19 75.58) (width 0.2) (layer "F.Cu") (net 9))
 (segment (start 116.11 42.39) (end 116.11 55.96) (width 0.2) (layer "F.Cu") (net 9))
 (segment (start 116.19 75.58) (end 116.15 75.54) (width 0.2) (layer "F.Cu") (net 9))
 (segment (start 122.92 35.58) (end 116.11 42.39) (width 0.2) (layer "F.Cu") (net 9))
 (segment (start 152.5 40) (end 155 37.5) (width 0.2) (layer "F.Cu") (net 6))
 (segment (start 152.5 40) (end 150.75 40) (width 0.2) (layer "F.Cu") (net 6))
 (segment (start 143.79 33.04) (end 142.455 33.04) (width 0.2) (layer "F.Cu") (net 6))
 (segment (start 155 37.5) (end 167 37.5) (width 0.2) (layer "F.Cu") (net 6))
 (segment (start 150.75 40) (end 143.79 33.04) (width 0.2) (layer "F.Cu") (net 6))
 (segment (start 143.75325 43.2) (end 142.455 43.2) (width 0.2) (layer "F.Cu") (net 7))
 (segment (start 165.25 44.25) (end 151.3171 44.25) (width 0.2) (layer "F.Cu") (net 7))
 (segment (start 146.00475 45.4515) (end 143.75325 43.2) (width 0.2) (layer "F.Cu") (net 7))
 (segment (start 150.1156 45.4515) (end 146.00475 45.4515) (width 0.2) (layer "F.Cu") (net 7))
 (segment (start 167 42.5) (end 165.25 44.25) (width 0.2) (layer "F.Cu") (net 7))
 (segment (start 151.3171 44.25) (end 150.1156 45.4515) (width 0.2) (layer "F.Cu") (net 7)))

